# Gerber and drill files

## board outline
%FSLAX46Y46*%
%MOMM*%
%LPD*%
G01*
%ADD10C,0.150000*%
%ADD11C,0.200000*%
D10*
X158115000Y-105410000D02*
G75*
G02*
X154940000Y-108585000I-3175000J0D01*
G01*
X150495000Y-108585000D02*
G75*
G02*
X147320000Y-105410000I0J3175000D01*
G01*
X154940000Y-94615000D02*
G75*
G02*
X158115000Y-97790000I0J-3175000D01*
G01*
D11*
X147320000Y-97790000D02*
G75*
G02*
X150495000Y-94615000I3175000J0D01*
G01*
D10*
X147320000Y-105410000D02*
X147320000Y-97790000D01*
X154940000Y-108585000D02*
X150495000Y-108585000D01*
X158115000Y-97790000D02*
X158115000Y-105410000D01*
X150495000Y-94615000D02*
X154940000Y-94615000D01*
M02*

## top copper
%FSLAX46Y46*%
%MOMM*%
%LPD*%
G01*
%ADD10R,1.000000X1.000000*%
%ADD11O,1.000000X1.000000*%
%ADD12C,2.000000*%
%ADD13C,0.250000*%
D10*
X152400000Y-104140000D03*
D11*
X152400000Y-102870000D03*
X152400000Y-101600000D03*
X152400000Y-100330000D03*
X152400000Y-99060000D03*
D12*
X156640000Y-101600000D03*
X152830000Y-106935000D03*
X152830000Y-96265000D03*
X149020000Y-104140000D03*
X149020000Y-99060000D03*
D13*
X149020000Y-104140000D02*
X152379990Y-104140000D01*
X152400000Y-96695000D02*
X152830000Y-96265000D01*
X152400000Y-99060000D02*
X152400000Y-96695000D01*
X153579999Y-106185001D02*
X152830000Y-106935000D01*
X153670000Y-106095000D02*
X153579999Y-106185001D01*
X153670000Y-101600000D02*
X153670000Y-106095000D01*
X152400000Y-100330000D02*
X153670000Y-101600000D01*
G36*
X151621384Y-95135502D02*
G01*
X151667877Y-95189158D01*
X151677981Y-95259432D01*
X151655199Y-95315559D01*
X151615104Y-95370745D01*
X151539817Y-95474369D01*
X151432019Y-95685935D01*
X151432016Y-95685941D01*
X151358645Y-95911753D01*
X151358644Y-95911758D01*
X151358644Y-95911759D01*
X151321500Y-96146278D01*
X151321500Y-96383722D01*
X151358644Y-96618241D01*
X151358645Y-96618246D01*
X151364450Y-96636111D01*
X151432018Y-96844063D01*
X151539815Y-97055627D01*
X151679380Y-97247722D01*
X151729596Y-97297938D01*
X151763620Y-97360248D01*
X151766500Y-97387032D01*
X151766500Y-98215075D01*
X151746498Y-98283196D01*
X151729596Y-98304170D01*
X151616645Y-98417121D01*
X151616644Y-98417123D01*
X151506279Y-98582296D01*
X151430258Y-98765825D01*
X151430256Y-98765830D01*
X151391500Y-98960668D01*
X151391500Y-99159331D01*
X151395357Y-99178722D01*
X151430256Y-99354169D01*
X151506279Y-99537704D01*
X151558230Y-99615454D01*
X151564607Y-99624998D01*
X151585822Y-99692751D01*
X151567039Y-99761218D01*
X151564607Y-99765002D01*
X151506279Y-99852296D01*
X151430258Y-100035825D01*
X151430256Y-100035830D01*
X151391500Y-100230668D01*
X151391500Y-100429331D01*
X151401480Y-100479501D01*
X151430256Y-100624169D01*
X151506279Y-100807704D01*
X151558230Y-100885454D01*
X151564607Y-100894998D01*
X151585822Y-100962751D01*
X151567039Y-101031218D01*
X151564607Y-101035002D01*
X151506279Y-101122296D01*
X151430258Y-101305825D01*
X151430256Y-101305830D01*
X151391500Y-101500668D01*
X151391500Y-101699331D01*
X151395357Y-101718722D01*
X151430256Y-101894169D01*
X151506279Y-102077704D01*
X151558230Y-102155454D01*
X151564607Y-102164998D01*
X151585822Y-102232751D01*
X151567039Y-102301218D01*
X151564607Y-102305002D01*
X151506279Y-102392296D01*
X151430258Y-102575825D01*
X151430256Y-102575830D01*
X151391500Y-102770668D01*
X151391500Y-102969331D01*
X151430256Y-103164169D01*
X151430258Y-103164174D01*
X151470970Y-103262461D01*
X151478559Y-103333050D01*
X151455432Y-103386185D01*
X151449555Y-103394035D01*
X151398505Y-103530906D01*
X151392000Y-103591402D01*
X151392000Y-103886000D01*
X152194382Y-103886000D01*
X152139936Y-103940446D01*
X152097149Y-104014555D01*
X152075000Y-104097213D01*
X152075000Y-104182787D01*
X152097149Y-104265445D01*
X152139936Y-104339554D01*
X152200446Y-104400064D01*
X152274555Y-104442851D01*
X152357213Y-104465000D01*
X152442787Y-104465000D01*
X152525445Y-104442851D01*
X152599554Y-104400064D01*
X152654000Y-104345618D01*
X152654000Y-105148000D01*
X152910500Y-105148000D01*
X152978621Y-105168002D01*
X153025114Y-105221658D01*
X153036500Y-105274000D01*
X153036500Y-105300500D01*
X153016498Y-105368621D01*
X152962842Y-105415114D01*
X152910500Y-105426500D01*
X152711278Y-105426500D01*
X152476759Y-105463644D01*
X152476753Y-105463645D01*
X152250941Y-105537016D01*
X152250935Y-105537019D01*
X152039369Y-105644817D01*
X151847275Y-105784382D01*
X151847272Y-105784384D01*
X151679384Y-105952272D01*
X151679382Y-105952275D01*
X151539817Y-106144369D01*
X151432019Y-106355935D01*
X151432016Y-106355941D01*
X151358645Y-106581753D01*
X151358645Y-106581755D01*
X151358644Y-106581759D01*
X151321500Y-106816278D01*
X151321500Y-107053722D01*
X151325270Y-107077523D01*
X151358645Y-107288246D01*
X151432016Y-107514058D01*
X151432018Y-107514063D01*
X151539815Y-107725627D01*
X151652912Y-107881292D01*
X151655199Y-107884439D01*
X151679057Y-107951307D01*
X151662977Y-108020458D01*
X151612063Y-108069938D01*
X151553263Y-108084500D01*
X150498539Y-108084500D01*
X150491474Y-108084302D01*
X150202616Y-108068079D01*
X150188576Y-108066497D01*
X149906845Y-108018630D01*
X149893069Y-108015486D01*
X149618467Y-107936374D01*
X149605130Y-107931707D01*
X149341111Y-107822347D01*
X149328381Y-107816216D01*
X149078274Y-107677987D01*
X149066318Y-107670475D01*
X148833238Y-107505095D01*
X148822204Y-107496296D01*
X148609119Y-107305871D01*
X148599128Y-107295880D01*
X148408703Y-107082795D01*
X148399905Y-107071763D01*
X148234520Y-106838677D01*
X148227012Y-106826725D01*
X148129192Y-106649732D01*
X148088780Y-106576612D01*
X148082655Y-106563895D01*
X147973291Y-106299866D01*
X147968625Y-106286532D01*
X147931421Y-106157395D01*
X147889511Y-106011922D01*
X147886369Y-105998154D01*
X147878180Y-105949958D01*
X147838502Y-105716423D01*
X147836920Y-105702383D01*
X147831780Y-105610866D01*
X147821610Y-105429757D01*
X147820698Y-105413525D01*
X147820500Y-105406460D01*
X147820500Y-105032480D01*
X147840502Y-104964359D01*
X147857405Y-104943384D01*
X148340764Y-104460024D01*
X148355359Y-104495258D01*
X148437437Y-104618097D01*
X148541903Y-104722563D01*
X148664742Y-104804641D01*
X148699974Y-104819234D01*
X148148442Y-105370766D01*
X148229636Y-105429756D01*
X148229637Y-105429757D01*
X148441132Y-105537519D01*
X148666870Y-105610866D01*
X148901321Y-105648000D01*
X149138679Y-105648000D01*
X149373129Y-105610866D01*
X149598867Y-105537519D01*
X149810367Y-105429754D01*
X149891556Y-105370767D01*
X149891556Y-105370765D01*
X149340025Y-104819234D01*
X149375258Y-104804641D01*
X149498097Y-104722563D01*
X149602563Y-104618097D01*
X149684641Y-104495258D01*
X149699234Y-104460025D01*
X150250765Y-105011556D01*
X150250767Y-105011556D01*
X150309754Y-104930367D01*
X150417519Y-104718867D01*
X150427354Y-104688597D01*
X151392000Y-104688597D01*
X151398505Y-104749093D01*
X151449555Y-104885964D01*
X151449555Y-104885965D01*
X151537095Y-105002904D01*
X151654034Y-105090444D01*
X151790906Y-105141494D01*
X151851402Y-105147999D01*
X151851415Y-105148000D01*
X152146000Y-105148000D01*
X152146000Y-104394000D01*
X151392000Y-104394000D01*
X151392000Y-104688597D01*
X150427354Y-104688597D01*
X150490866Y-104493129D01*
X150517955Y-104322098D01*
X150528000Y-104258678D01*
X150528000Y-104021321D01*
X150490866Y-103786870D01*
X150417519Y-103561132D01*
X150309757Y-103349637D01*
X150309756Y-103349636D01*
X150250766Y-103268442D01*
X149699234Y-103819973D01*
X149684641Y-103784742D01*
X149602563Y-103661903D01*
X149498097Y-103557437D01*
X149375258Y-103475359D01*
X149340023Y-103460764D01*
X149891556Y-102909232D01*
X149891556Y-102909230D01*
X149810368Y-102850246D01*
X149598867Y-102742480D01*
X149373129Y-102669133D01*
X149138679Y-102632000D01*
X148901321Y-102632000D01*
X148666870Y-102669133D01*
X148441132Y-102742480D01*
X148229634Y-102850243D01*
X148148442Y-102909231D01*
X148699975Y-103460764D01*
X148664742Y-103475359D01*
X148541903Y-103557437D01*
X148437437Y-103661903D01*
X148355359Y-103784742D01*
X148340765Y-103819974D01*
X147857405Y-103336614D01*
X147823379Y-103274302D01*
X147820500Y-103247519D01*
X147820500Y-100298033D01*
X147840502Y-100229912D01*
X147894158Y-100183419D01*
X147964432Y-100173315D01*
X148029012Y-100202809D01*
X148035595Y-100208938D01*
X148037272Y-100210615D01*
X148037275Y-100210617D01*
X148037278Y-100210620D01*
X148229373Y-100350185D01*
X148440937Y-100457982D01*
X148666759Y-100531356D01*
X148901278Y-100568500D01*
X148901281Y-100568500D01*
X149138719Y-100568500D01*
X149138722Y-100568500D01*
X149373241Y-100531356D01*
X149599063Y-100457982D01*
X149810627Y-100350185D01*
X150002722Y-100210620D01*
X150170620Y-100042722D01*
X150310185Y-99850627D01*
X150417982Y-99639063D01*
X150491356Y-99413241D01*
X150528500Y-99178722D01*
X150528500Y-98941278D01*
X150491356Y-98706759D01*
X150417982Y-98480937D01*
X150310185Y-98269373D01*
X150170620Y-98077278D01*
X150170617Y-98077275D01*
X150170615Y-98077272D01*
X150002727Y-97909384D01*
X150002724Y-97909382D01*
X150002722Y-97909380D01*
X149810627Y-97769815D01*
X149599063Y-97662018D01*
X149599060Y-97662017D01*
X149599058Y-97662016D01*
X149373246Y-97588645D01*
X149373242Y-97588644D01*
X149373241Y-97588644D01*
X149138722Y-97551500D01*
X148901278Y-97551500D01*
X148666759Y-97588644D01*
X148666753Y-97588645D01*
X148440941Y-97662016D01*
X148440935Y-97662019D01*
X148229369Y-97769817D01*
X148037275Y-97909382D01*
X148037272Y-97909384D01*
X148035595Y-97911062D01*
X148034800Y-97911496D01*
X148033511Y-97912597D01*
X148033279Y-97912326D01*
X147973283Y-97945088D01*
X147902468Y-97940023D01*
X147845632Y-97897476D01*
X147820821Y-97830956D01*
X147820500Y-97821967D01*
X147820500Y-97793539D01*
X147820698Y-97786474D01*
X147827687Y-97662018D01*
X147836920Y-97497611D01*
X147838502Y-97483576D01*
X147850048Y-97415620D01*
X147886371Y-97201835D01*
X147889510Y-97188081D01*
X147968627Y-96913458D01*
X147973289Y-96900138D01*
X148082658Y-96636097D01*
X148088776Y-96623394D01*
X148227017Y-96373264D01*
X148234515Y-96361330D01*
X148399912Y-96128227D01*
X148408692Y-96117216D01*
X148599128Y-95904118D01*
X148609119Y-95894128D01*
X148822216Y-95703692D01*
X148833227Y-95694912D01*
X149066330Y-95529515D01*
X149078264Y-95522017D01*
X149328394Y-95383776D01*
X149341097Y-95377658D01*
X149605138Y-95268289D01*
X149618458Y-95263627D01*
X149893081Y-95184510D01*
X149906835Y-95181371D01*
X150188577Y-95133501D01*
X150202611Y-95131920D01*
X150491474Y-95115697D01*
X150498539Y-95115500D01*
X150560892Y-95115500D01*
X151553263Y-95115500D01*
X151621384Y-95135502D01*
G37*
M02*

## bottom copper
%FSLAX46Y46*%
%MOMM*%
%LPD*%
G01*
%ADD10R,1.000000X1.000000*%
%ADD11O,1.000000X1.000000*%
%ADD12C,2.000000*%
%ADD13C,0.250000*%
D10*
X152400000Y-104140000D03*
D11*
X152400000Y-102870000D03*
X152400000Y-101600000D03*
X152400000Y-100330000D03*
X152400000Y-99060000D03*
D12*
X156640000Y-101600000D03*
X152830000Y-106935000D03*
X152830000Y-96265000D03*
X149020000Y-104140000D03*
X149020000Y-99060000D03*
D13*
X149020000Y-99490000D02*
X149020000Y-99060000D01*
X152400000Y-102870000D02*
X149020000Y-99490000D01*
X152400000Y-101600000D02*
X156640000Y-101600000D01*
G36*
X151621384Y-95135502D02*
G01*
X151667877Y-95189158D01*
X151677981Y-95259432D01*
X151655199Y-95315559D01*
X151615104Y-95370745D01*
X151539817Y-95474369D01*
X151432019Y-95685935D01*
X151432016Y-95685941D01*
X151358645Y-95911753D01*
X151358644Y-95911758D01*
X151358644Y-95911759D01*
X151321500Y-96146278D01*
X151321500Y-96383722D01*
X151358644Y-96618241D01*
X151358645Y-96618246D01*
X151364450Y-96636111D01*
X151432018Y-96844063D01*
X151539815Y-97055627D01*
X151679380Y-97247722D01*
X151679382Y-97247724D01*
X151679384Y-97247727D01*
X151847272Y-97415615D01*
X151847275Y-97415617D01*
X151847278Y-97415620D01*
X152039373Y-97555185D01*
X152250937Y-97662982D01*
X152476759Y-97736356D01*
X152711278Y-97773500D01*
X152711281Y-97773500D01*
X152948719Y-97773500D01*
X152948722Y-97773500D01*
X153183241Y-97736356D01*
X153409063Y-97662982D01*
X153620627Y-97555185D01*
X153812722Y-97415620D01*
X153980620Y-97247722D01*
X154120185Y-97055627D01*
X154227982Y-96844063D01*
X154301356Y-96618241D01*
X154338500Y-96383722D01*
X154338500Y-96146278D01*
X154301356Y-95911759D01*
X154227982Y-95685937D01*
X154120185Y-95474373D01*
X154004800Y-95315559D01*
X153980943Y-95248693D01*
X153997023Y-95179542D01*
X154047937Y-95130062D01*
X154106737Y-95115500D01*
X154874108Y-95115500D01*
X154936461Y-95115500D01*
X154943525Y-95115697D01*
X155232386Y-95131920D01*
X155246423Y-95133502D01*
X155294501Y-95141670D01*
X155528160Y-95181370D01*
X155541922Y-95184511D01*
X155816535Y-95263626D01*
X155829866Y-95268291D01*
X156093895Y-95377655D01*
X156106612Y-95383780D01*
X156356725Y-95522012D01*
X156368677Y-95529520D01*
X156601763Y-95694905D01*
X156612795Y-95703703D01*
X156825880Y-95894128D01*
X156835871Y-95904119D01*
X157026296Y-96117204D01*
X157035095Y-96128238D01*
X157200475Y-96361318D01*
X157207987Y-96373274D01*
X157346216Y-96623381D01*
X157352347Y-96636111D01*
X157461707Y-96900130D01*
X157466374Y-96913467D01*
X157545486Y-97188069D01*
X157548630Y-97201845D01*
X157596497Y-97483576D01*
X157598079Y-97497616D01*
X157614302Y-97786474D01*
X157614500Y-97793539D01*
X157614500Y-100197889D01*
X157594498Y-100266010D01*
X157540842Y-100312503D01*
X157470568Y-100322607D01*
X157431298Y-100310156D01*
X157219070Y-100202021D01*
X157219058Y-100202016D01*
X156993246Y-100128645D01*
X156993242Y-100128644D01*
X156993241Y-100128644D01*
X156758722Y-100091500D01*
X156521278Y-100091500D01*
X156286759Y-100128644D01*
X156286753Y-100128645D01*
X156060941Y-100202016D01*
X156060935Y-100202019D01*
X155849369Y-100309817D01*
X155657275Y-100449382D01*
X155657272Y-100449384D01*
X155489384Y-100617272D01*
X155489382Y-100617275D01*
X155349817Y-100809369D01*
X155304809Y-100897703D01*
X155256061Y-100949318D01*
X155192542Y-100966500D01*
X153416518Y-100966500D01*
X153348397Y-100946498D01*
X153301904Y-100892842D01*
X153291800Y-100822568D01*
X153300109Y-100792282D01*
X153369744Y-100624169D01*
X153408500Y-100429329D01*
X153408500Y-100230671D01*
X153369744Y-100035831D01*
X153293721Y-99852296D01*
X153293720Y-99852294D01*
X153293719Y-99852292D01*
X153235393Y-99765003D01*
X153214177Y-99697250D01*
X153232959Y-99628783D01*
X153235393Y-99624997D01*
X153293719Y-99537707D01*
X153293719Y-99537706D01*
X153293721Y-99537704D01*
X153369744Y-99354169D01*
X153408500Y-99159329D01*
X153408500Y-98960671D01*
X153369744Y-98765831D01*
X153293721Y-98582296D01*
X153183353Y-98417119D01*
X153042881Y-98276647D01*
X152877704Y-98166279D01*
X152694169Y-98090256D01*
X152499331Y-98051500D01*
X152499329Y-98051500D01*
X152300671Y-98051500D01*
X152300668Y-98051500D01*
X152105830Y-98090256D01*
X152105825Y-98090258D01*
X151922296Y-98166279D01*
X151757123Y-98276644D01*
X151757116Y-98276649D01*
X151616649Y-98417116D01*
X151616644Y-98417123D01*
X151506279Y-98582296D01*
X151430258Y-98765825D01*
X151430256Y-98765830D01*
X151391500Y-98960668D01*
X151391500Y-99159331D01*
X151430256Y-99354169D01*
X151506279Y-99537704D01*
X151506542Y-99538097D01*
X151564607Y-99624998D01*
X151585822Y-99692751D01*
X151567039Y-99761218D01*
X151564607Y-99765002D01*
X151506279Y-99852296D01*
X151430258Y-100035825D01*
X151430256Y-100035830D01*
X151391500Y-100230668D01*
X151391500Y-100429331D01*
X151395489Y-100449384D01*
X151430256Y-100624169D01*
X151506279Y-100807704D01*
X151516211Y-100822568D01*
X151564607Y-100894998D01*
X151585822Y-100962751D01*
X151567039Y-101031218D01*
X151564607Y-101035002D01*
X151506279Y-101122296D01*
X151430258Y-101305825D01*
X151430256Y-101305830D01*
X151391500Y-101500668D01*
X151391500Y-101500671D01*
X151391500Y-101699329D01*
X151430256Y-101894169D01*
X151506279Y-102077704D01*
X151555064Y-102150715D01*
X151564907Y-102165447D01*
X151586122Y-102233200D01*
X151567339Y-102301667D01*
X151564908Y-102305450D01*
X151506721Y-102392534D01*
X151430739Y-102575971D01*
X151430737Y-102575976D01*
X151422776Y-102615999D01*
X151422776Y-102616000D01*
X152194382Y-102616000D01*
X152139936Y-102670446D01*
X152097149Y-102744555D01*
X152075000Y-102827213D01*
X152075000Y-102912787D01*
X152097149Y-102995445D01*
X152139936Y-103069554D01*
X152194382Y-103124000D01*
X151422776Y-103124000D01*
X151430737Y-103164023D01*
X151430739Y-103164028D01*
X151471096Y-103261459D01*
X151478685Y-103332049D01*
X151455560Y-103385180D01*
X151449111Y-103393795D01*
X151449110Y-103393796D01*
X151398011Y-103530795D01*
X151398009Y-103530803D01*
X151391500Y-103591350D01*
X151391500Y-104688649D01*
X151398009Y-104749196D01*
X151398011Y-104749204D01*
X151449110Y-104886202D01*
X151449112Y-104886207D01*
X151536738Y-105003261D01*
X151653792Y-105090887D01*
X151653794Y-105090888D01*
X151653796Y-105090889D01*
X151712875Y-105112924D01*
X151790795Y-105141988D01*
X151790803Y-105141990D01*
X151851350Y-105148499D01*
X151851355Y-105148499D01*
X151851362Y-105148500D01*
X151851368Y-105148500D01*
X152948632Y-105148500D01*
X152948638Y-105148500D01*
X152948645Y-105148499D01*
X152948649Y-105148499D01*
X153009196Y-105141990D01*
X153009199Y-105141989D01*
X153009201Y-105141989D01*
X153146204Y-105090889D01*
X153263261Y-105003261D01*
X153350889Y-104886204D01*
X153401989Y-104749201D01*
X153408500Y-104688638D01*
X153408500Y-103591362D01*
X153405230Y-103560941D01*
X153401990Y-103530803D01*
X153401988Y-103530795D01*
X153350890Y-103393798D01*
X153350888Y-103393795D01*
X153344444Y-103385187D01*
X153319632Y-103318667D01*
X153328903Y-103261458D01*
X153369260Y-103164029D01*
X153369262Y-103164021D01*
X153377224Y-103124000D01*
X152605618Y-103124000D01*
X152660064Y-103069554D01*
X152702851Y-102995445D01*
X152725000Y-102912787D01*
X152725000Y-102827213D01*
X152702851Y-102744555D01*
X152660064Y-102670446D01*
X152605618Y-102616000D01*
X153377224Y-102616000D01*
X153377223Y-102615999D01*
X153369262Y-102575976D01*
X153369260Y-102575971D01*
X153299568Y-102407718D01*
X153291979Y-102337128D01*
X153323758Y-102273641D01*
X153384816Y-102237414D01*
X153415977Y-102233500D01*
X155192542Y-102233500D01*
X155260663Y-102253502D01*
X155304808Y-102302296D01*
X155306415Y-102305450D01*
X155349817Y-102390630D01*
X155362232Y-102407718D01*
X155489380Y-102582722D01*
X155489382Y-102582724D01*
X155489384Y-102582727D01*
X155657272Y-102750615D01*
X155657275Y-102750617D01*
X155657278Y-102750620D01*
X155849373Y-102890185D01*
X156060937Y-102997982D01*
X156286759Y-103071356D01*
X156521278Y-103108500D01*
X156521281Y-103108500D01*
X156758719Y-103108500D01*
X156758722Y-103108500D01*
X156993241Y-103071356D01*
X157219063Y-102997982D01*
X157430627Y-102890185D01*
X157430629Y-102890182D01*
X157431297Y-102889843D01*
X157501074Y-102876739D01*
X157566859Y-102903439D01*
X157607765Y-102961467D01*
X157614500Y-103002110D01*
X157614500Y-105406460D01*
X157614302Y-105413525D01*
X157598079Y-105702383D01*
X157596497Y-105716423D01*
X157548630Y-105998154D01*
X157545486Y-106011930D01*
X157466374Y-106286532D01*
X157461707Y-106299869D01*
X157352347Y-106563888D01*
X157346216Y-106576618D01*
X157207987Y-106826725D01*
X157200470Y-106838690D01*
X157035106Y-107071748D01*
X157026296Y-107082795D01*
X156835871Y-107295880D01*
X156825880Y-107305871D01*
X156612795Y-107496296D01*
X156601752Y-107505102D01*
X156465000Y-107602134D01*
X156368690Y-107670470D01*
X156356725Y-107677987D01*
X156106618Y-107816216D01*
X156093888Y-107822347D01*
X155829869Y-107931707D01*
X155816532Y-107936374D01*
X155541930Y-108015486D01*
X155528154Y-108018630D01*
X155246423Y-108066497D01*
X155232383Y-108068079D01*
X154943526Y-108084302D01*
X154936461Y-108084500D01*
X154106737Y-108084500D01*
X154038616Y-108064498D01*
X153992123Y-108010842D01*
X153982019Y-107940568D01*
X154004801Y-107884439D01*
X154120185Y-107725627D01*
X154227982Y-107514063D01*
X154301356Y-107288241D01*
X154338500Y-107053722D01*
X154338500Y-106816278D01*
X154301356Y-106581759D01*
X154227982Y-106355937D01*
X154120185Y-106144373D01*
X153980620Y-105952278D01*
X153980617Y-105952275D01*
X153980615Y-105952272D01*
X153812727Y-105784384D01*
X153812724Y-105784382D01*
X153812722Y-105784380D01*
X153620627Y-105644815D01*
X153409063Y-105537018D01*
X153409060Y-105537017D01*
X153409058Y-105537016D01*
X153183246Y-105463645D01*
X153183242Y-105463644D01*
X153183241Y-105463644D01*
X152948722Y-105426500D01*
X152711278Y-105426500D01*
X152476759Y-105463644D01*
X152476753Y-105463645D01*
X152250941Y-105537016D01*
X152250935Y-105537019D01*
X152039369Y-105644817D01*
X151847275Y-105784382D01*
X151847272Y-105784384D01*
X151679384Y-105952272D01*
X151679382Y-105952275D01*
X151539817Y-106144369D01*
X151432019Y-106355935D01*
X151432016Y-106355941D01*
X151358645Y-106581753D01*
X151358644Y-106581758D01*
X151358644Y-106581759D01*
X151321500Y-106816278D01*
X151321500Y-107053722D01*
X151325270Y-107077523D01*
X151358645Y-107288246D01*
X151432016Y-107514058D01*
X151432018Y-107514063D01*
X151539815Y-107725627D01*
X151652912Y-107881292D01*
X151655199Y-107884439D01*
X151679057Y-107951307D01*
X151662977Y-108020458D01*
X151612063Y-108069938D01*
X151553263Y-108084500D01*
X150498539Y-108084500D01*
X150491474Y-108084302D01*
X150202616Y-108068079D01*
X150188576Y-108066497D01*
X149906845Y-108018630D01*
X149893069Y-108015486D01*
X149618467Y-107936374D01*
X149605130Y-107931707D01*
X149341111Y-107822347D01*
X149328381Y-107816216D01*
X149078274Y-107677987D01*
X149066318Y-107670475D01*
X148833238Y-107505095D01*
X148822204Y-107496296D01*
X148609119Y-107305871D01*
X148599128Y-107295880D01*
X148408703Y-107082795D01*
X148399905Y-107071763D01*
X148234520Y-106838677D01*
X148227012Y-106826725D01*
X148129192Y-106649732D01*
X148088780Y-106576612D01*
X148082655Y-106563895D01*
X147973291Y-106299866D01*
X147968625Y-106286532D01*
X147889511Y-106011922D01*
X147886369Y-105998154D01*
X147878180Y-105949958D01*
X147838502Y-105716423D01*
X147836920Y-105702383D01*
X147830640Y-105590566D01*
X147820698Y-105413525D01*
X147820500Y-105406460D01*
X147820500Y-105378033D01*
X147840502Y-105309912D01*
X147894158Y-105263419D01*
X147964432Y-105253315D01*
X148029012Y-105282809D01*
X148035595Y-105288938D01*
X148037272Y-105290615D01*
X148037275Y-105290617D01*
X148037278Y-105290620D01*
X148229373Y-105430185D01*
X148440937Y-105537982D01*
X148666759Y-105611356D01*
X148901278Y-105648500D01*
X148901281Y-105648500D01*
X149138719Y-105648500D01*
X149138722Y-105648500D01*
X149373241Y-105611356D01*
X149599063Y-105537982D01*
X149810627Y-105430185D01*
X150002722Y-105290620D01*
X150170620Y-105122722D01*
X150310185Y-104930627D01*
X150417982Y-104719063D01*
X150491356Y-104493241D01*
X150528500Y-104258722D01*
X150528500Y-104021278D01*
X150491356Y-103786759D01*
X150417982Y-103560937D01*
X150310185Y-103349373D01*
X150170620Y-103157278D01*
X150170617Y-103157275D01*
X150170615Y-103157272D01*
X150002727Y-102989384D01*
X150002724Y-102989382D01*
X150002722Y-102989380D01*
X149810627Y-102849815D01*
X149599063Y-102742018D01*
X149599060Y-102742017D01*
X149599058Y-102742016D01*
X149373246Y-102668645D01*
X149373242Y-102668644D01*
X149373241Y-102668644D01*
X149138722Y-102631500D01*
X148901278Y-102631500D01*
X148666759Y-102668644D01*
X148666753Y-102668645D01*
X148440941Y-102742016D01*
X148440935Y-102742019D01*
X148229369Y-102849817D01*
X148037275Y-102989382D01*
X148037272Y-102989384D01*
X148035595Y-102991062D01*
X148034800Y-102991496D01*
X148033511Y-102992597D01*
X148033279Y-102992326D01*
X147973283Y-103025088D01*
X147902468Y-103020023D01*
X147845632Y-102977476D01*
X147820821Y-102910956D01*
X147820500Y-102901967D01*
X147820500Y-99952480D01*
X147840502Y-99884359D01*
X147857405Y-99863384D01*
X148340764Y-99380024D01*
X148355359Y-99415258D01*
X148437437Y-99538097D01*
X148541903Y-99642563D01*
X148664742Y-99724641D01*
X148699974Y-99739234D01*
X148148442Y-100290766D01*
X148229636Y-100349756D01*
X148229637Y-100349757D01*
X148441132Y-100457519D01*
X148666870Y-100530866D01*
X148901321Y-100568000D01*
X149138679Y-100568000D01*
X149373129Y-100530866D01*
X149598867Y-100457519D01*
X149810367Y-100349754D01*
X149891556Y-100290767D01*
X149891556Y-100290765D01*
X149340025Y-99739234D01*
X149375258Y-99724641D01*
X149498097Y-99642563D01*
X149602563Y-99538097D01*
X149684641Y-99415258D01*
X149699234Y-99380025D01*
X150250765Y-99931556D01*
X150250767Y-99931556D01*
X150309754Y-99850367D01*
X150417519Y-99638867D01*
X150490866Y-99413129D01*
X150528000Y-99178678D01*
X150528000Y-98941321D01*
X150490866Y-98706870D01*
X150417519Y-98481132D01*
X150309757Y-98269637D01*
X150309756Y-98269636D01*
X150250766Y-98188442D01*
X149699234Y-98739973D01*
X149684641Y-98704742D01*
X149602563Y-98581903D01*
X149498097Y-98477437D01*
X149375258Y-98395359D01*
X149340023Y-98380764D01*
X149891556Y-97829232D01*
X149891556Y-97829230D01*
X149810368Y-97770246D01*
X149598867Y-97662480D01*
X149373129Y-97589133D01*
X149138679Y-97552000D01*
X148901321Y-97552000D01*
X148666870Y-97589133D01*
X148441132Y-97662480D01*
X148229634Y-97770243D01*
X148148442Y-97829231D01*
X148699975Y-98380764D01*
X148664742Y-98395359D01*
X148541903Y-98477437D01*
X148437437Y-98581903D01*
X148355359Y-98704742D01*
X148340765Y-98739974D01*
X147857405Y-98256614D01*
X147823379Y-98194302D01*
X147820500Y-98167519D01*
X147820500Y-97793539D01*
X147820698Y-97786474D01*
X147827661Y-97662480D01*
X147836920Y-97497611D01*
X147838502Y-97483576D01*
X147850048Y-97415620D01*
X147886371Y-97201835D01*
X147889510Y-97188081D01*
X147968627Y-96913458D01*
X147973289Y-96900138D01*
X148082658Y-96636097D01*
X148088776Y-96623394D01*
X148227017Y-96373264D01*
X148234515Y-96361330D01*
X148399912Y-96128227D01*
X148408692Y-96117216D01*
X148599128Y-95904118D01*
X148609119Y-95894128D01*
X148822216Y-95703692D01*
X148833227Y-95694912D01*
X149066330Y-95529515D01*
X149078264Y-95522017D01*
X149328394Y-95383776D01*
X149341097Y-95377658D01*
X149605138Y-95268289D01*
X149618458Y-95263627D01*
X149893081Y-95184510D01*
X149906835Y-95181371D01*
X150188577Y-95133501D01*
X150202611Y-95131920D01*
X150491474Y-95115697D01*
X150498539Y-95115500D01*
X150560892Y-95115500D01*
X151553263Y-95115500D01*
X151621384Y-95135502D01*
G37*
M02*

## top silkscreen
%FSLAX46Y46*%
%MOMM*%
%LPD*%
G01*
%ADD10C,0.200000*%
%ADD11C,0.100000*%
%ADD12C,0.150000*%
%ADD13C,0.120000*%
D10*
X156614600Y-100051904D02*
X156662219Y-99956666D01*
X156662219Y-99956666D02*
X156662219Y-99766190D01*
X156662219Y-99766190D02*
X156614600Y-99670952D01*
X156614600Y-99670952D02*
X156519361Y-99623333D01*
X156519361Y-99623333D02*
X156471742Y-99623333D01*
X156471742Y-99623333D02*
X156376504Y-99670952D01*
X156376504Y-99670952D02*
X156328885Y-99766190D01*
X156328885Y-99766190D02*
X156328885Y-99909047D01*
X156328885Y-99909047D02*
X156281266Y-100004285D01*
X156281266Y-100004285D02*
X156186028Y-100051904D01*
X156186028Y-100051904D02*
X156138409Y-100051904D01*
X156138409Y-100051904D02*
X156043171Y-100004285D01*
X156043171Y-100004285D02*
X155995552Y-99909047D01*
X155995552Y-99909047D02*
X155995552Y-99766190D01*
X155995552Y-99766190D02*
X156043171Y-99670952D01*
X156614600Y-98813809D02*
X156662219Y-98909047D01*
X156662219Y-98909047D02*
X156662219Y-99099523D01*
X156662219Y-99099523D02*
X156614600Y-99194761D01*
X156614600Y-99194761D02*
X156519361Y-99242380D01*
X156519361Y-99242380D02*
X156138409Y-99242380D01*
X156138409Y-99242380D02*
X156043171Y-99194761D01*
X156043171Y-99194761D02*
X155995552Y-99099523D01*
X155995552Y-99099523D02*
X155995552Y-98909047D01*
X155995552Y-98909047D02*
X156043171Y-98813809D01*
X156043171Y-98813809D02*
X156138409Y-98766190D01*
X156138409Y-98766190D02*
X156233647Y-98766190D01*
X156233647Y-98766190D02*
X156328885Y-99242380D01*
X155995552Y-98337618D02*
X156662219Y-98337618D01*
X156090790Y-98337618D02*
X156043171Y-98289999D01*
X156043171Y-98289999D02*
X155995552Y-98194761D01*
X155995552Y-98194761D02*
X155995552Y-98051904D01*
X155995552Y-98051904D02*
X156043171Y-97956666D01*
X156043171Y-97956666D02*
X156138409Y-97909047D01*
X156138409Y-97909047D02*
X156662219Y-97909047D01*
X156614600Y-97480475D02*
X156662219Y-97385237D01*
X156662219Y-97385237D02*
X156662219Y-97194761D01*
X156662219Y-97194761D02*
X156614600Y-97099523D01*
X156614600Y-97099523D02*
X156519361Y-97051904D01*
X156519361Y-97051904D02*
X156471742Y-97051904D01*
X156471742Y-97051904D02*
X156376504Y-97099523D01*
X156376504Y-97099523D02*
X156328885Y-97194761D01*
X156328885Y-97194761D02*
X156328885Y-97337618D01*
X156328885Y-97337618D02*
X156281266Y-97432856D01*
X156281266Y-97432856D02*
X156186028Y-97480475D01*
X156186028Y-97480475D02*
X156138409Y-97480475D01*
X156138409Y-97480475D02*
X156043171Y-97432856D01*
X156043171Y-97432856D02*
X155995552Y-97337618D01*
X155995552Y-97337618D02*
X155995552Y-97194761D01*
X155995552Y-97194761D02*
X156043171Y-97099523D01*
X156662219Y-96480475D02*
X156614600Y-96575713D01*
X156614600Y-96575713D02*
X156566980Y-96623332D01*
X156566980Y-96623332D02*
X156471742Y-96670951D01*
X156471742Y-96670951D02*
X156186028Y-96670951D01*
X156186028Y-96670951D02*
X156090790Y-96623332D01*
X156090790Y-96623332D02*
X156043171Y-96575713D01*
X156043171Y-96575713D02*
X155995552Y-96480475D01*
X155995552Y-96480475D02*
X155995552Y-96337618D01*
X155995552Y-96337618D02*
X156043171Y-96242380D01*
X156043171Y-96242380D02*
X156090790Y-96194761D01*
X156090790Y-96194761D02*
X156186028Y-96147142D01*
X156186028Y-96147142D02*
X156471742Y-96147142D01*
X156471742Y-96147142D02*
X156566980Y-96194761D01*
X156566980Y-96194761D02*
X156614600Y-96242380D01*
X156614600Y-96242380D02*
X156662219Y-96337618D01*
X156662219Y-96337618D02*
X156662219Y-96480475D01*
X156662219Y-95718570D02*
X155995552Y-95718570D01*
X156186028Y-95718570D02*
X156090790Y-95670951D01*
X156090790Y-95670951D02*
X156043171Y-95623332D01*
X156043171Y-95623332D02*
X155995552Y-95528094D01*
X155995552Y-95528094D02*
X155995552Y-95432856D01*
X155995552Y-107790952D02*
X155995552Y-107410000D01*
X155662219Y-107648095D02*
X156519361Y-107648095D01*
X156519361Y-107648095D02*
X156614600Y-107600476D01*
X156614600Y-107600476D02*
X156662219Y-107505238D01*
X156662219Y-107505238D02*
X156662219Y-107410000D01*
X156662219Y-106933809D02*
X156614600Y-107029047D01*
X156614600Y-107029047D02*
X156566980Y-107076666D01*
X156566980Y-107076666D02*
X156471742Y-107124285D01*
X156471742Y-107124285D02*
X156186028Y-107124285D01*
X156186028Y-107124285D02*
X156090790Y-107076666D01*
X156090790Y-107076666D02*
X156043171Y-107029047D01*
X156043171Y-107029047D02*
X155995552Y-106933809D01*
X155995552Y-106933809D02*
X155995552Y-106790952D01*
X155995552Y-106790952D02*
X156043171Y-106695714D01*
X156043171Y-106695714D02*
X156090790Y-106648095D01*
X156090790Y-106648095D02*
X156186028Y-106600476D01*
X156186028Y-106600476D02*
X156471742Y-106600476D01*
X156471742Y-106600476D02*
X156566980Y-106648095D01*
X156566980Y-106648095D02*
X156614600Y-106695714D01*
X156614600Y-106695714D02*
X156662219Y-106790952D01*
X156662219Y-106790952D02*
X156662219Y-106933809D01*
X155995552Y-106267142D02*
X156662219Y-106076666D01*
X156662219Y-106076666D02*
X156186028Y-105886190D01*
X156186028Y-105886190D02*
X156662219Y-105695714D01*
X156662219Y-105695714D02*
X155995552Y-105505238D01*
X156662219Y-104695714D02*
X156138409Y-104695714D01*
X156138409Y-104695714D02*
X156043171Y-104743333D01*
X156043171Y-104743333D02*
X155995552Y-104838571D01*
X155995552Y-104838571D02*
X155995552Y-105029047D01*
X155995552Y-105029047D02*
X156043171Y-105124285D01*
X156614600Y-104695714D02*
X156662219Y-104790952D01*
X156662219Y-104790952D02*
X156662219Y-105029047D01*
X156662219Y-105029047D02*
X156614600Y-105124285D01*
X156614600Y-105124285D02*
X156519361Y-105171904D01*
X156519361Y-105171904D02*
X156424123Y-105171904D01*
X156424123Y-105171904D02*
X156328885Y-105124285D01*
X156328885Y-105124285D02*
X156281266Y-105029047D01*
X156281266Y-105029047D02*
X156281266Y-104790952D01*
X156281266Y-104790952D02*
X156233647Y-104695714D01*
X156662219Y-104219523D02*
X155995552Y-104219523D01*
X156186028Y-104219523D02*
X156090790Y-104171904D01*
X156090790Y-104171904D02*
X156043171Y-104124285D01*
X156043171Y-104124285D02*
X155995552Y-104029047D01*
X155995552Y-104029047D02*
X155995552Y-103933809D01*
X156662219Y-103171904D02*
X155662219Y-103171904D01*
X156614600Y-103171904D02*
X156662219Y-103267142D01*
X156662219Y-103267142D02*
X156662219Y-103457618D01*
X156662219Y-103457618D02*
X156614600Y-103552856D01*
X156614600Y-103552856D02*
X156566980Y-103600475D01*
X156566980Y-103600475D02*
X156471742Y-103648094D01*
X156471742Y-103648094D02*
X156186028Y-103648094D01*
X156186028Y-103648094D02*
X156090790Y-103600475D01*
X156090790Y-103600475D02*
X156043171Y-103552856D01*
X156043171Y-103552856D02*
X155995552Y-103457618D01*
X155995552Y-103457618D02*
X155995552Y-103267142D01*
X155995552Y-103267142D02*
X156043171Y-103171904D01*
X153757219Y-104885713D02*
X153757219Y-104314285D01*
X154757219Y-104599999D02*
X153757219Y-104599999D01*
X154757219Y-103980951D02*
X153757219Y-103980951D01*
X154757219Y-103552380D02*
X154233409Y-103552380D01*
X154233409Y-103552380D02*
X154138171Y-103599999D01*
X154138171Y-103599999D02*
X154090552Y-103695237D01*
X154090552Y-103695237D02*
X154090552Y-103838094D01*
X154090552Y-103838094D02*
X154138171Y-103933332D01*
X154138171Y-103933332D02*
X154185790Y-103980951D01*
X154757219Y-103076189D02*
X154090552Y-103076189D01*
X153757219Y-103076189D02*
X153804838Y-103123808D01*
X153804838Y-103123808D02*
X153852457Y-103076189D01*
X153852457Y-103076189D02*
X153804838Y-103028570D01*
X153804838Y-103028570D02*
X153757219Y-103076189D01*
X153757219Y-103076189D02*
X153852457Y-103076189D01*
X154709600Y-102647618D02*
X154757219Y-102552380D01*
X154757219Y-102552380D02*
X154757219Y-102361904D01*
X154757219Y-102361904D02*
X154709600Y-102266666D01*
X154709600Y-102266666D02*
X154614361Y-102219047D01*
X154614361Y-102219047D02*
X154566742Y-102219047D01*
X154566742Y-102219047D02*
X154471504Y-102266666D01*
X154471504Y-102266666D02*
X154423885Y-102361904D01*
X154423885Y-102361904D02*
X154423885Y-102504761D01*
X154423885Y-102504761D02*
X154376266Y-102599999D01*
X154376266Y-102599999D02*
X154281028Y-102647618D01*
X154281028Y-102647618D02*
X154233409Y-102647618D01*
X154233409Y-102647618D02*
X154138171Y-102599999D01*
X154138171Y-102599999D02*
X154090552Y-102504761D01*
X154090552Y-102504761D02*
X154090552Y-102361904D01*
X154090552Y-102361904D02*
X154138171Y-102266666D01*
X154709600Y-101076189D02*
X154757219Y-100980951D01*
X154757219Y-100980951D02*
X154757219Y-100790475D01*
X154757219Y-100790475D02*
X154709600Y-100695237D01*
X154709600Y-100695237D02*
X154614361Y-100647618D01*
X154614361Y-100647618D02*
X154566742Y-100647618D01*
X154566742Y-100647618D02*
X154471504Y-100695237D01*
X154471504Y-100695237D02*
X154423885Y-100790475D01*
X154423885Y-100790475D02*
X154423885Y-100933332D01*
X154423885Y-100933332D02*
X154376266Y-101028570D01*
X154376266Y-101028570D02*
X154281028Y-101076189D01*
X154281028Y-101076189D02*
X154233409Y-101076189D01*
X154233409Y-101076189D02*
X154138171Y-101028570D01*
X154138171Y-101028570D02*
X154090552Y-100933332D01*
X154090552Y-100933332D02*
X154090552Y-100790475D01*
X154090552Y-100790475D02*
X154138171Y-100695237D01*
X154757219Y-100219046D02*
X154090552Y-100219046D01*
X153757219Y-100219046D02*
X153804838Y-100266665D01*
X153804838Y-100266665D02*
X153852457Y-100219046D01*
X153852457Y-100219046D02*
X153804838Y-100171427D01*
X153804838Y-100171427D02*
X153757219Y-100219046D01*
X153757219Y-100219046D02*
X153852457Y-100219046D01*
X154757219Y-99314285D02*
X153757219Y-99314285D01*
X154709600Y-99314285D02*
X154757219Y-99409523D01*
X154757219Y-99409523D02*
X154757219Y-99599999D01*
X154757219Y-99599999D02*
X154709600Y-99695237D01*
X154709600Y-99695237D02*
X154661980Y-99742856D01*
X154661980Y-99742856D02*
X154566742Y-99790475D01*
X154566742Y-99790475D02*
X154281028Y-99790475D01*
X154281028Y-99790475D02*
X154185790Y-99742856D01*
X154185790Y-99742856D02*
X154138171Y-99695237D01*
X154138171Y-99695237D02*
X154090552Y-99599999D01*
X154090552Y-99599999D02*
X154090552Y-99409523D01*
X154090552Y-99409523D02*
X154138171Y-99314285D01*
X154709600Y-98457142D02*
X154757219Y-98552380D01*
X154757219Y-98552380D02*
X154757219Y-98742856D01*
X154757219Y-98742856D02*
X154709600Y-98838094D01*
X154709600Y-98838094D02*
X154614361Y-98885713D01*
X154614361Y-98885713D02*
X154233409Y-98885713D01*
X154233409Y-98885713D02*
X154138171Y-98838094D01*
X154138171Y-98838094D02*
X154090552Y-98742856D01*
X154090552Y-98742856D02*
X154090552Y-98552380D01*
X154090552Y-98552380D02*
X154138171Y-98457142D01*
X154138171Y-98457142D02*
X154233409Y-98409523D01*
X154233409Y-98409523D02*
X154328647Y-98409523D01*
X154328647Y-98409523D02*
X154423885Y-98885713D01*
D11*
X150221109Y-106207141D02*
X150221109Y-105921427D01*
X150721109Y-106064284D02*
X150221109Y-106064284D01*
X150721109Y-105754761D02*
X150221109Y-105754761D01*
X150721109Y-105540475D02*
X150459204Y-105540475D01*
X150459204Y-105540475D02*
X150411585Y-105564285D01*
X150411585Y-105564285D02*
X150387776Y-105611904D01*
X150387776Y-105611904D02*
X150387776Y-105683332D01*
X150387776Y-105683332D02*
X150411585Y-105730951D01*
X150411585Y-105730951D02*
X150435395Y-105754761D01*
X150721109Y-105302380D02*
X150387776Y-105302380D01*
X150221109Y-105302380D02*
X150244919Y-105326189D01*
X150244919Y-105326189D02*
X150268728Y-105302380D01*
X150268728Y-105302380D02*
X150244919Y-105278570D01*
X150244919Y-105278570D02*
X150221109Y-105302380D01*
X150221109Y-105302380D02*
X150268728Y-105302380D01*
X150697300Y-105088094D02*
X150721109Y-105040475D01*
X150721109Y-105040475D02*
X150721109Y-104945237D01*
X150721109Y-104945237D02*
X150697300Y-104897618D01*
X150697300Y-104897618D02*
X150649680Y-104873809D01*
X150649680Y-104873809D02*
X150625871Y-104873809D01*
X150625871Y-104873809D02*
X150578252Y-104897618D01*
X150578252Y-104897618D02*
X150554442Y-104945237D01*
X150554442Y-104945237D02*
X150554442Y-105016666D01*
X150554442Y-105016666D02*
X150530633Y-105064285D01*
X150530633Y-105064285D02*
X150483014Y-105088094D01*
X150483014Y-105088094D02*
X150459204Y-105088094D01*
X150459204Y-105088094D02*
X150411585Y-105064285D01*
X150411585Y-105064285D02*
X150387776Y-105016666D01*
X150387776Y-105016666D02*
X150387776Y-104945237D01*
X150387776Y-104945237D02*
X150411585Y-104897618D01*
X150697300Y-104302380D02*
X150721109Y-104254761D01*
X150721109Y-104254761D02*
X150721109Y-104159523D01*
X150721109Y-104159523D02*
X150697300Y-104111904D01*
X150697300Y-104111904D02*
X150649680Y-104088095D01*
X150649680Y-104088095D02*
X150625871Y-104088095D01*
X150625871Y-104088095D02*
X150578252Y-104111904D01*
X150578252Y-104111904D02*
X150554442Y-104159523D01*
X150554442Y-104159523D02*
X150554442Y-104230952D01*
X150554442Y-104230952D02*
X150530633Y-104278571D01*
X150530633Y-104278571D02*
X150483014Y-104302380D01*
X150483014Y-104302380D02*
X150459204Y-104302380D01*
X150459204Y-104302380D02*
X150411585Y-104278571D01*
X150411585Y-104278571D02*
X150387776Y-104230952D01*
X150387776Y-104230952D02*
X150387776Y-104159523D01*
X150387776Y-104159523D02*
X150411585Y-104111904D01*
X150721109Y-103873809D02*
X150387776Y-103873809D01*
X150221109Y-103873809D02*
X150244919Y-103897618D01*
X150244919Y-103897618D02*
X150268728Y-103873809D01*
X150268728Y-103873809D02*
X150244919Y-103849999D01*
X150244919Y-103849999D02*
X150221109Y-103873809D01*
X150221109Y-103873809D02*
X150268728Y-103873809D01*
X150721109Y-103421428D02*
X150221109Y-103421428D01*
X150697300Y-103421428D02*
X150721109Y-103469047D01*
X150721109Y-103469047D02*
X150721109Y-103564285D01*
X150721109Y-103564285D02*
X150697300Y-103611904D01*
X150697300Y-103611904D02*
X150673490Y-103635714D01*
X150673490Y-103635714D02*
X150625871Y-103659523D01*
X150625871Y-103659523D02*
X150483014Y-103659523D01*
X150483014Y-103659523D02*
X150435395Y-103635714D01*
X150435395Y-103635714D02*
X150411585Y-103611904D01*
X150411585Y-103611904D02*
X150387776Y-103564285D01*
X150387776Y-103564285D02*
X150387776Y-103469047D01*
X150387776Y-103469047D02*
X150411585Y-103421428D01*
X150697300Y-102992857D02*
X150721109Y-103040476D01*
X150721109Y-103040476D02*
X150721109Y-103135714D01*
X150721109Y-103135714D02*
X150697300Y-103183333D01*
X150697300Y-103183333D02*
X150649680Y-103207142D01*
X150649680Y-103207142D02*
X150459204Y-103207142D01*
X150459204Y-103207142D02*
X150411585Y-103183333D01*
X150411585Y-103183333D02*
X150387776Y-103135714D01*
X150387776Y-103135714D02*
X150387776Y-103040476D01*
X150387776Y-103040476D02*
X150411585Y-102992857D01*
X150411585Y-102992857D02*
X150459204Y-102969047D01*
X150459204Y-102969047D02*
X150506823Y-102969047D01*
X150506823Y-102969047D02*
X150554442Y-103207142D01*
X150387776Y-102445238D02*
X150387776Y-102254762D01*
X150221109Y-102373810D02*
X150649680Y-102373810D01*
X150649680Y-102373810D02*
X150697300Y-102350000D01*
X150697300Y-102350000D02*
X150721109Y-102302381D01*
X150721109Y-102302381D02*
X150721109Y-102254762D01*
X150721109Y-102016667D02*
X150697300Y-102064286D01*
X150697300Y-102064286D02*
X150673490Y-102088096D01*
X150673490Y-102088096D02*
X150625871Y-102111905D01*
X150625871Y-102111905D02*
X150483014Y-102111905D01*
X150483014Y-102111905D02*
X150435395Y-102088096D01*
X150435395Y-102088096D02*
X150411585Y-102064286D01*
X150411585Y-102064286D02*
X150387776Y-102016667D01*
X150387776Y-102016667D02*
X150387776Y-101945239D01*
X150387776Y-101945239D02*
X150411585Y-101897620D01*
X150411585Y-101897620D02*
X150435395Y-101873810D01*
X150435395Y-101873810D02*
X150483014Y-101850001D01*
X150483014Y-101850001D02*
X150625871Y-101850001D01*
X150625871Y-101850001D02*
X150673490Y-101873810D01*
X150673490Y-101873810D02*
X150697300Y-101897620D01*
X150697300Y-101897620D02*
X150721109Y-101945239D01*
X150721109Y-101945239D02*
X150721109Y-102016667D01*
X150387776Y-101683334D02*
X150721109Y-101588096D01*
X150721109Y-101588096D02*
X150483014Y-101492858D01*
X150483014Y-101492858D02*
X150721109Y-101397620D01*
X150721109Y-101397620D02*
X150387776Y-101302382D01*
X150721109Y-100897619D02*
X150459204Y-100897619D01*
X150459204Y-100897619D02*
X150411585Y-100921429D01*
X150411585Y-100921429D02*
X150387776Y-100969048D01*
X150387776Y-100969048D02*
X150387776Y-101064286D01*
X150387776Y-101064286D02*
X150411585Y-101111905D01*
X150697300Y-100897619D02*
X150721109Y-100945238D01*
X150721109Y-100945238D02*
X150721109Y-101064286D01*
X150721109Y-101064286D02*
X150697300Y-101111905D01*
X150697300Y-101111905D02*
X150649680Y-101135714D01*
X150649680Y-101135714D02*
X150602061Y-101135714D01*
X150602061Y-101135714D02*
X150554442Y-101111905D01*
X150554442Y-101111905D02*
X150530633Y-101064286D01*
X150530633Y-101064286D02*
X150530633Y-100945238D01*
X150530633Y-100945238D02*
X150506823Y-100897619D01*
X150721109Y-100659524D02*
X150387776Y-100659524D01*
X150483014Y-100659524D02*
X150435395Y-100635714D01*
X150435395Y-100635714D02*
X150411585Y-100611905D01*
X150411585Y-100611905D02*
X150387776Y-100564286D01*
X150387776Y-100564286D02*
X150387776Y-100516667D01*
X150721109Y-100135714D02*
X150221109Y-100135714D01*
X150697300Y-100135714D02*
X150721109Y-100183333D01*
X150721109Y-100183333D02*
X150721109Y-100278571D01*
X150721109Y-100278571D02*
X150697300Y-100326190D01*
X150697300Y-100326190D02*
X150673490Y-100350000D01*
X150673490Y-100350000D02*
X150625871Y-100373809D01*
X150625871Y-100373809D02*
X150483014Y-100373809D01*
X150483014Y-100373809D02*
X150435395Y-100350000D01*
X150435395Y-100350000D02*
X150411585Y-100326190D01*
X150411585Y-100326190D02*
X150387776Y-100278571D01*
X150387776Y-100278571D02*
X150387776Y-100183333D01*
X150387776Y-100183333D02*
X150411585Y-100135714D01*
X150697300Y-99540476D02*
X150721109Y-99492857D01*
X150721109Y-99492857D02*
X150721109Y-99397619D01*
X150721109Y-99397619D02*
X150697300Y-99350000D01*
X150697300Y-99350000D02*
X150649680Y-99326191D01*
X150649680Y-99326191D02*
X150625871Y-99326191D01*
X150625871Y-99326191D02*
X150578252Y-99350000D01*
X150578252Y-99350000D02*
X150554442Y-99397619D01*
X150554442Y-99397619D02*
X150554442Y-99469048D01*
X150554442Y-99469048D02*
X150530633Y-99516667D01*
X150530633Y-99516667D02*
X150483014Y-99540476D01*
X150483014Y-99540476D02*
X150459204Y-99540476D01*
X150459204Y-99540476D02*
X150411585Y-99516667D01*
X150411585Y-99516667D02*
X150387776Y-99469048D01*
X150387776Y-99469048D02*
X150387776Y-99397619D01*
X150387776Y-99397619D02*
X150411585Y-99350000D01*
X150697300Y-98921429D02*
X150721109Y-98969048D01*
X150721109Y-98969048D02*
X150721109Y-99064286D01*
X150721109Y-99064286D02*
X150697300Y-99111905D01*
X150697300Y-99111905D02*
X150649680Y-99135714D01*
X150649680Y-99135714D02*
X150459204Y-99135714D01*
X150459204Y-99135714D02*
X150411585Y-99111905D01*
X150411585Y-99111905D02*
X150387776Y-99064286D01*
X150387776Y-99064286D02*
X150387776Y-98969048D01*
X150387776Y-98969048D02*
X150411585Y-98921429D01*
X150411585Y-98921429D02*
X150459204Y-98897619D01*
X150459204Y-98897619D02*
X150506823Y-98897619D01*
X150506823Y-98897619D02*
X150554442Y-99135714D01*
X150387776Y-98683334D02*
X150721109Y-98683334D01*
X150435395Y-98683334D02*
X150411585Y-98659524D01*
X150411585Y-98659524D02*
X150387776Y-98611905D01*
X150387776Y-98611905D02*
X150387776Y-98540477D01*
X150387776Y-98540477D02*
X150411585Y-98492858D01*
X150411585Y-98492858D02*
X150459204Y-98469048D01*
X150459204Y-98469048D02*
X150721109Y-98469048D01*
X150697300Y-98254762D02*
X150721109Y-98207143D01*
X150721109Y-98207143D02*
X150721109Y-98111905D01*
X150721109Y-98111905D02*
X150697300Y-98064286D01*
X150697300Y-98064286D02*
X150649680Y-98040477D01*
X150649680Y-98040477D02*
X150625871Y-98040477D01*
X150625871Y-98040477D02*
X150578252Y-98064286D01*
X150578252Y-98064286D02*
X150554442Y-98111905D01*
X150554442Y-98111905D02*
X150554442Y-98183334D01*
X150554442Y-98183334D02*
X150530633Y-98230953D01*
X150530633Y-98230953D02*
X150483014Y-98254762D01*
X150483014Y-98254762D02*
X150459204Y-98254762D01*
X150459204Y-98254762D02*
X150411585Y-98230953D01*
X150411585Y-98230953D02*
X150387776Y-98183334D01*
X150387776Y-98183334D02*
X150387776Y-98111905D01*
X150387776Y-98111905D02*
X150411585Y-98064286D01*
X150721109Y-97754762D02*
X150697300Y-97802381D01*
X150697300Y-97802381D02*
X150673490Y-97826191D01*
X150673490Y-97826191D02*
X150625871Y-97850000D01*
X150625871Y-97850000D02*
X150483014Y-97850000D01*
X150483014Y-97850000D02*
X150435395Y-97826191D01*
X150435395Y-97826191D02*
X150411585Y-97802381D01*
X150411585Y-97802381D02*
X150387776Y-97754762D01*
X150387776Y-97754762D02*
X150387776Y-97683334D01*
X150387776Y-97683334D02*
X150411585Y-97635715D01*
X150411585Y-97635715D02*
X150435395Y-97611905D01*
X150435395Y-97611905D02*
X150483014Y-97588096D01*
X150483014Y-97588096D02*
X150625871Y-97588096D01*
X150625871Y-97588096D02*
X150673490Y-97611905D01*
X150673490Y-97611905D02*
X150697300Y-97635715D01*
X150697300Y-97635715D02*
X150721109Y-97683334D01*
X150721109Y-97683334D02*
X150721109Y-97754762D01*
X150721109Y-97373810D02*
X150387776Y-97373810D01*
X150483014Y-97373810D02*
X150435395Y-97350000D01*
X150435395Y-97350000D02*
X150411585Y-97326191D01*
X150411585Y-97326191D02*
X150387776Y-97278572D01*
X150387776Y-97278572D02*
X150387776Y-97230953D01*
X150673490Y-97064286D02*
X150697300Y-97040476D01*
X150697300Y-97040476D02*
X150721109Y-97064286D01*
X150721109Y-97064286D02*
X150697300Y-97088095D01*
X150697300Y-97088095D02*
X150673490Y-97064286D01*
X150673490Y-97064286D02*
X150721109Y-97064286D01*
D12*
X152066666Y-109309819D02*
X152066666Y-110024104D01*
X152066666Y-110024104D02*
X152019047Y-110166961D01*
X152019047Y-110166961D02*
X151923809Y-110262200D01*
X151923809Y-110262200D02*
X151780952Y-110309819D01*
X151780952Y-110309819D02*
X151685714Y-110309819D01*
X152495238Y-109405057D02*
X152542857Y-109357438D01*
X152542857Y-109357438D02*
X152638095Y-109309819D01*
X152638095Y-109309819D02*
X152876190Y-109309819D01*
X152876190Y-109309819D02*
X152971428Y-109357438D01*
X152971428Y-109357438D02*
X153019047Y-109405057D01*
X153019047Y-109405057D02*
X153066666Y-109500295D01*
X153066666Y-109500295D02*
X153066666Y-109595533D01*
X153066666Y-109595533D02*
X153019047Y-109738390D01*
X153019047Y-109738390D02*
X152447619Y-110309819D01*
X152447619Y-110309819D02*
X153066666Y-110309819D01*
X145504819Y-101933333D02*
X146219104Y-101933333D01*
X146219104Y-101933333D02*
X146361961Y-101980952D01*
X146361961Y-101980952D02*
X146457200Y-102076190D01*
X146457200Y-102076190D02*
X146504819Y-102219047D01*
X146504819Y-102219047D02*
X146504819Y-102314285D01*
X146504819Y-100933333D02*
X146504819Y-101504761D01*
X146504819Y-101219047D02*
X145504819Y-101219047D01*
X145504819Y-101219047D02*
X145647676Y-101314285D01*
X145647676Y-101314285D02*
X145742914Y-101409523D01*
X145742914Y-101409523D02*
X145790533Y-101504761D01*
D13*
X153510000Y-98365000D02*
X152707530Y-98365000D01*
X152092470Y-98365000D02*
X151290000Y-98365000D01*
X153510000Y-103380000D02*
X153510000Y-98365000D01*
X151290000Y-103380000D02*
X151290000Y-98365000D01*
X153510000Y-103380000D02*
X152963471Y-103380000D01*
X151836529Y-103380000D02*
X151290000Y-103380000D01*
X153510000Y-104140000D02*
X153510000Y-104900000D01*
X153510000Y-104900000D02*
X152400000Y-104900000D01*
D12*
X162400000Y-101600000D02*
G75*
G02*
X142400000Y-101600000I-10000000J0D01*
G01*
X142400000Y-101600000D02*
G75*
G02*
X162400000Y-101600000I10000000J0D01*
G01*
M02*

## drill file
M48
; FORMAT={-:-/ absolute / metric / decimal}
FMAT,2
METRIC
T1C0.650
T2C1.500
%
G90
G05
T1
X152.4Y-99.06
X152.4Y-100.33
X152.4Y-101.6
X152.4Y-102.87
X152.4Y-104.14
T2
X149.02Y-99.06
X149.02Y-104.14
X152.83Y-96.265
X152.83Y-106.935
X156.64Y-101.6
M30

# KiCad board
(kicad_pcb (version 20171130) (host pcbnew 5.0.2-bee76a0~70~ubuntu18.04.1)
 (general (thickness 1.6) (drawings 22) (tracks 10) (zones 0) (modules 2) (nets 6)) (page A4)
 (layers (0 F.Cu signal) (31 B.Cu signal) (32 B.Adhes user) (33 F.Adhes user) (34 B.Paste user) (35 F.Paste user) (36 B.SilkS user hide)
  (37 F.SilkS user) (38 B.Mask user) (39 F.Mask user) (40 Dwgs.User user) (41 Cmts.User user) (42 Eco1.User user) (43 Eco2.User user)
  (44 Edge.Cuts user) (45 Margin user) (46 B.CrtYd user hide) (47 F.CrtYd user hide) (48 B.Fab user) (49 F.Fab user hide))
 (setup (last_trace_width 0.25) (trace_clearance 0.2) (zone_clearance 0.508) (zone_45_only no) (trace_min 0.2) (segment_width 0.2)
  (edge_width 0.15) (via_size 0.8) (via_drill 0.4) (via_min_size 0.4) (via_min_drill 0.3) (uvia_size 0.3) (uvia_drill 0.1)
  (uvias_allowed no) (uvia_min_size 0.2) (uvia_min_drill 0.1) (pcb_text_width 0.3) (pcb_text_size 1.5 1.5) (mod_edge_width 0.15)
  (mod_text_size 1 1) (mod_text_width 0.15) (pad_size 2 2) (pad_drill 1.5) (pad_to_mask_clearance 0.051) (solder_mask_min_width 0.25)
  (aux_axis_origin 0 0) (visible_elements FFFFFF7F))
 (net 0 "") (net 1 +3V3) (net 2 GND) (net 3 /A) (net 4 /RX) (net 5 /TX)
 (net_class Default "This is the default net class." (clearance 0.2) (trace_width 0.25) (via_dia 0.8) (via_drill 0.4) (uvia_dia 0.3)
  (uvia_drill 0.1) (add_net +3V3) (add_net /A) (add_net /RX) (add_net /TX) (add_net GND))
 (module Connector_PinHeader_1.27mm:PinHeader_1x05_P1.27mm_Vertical (layer F.Cu) (at 152.4 104.14 180)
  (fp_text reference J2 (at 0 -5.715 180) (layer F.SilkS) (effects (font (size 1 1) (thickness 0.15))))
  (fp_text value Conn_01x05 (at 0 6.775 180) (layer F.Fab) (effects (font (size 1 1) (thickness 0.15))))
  (fp_line (start -1.11 5.775) (end -0.30753 5.775) (layer F.SilkS) (width 0.12))
  (fp_line (start 0.30753 5.775) (end 1.11 5.775) (layer F.SilkS) (width 0.12))
  (fp_line (start -1.11 0.76) (end -1.11 5.775) (layer F.SilkS) (width 0.12))
  (fp_line (start 1.11 0.76) (end 1.11 5.775) (layer F.SilkS) (width 0.12))
  (fp_line (start -1.11 0.76) (end -0.563471 0.76) (layer F.SilkS) (width 0.12))
  (fp_line (start 0.563471 0.76) (end 1.11 0.76) (layer F.SilkS) (width 0.12))
  (fp_line (start -1.11 0) (end -1.11 -0.76) (layer F.SilkS) (width 0.12))
  (fp_line (start -1.11 -0.76) (end 0 -0.76) (layer F.SilkS) (width 0.12))
  (pad 1 thru_hole rect (at 0 0 180) (size 1 1) (drill 0.65) (layers *.Cu *.Mask) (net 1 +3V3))
  (pad 2 thru_hole oval (at 0 1.27 180) (size 1 1) (drill 0.65) (layers *.Cu *.Mask) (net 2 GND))
  (pad 3 thru_hole oval (at 0 2.54 180) (size 1 1) (drill 0.65) (layers *.Cu *.Mask) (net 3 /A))
  (pad 4 thru_hole oval (at 0 3.81 180) (size 1 1) (drill 0.65) (layers *.Cu *.Mask) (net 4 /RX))
  (pad 5 thru_hole oval (at 0 5.08 180) (size 1 1) (drill 0.65) (layers *.Cu *.Mask) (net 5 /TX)))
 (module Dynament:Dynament (layer F.Cu) (at 152.4 101.6 270)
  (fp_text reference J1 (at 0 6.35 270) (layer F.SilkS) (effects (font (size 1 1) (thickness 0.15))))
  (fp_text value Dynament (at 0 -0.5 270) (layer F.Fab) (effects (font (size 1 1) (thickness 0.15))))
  (fp_circle (center 0 0) (end 10 0) (layer F.SilkS) (width 0.15))
  (pad OUT thru_hole circle (at 0 -4.24 270) (size 2 2) (drill 1.5) (layers *.Cu *.Mask) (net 3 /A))
  (pad RX thru_hole circle (at 5.335 -0.43 270) (size 2 2) (drill 1.5) (layers *.Cu *.Mask) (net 4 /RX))
  (pad TX thru_hole circle (at -5.335 -0.43 270) (size 2 2) (drill 1.5) (layers *.Cu *.Mask) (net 5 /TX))
  (pad 3V3 thru_hole circle (at 2.54 3.38 270) (size 2 2) (drill 1.5) (layers *.Cu *.Mask) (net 1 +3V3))
  (pad GND thru_hole circle (at -2.54 3.38 270) (size 2 2) (drill 1.5) (layers *.Cu *.Mask) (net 2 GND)))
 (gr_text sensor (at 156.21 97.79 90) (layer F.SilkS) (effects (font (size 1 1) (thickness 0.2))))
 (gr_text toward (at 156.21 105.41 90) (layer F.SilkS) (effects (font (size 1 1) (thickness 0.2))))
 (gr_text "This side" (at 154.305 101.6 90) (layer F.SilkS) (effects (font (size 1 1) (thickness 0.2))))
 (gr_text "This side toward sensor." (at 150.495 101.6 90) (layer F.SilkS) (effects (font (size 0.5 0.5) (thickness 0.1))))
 (gr_arc (start 154.94 105.41) (end 154.94 108.585) (angle -90) (layer Edge.Cuts) (width 0.15))
 (gr_arc (start 150.495 105.41) (end 147.32 105.41) (angle -90) (layer Edge.Cuts) (width 0.15))
 (gr_arc (start 154.94 97.79) (end 158.115 97.79) (angle -90) (layer Edge.Cuts) (width 0.15))
 (gr_arc (start 150.495 97.79) (end 150.495 94.615) (angle -90) (layer Edge.Cuts) (width 0.2))
 (gr_line (start 147.32 105.41) (end 147.32 97.79) (layer Edge.Cuts) (width 0.15))
 (gr_line (start 154.94 108.585) (end 150.495 108.585) (layer Edge.Cuts) (width 0.15))
 (gr_line (start 158.115 97.79) (end 158.115 105.41) (layer Edge.Cuts) (width 0.15))
 (gr_line (start 150.495 94.615) (end 154.94 94.615) (layer Edge.Cuts) (width 0.15))
 (segment (start 149.02 104.14) (end 152.37999 104.14) (width 0.25) (layer F.Cu) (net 1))
 (segment (start 149.02 99.49) (end 149.02 99.06) (width 0.25) (layer B.Cu) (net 2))
 (segment (start 152.4 102.87) (end 149.02 99.49) (width 0.25) (layer B.Cu) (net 2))
 (segment (start 152.4 101.6) (end 156.64 101.6) (width 0.25) (layer B.Cu) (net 3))
 (segment (start 152.4 96.695) (end 152.83 96.265) (width 0.25) (layer F.Cu) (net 5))
 (segment (start 152.4 99.06) (end 152.4 96.695) (width 0.25) (layer F.Cu) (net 5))
 (segment (start 153.579999 106.185001) (end 152.83 106.935) (width 0.25) (layer F.Cu) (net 4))
 (segment (start 153.67 106.095) (end 153.579999 106.185001) (width 0.25) (layer F.Cu) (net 4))
 (segment (start 153.67 101.6) (end 153.67 106.095) (width 0.25) (layer F.Cu) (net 4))
 (segment (start 152.4 100.33) (end 153.67 101.6) (width 0.25) (layer F.Cu) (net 4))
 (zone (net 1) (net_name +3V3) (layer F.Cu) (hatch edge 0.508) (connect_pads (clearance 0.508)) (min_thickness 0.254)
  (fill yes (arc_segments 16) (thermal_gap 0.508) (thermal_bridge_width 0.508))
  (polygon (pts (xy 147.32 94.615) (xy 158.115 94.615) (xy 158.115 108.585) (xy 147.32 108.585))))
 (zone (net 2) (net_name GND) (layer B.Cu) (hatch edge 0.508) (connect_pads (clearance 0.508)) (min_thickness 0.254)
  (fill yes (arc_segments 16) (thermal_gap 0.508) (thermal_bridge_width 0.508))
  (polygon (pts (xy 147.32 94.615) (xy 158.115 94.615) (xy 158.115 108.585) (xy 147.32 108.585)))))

